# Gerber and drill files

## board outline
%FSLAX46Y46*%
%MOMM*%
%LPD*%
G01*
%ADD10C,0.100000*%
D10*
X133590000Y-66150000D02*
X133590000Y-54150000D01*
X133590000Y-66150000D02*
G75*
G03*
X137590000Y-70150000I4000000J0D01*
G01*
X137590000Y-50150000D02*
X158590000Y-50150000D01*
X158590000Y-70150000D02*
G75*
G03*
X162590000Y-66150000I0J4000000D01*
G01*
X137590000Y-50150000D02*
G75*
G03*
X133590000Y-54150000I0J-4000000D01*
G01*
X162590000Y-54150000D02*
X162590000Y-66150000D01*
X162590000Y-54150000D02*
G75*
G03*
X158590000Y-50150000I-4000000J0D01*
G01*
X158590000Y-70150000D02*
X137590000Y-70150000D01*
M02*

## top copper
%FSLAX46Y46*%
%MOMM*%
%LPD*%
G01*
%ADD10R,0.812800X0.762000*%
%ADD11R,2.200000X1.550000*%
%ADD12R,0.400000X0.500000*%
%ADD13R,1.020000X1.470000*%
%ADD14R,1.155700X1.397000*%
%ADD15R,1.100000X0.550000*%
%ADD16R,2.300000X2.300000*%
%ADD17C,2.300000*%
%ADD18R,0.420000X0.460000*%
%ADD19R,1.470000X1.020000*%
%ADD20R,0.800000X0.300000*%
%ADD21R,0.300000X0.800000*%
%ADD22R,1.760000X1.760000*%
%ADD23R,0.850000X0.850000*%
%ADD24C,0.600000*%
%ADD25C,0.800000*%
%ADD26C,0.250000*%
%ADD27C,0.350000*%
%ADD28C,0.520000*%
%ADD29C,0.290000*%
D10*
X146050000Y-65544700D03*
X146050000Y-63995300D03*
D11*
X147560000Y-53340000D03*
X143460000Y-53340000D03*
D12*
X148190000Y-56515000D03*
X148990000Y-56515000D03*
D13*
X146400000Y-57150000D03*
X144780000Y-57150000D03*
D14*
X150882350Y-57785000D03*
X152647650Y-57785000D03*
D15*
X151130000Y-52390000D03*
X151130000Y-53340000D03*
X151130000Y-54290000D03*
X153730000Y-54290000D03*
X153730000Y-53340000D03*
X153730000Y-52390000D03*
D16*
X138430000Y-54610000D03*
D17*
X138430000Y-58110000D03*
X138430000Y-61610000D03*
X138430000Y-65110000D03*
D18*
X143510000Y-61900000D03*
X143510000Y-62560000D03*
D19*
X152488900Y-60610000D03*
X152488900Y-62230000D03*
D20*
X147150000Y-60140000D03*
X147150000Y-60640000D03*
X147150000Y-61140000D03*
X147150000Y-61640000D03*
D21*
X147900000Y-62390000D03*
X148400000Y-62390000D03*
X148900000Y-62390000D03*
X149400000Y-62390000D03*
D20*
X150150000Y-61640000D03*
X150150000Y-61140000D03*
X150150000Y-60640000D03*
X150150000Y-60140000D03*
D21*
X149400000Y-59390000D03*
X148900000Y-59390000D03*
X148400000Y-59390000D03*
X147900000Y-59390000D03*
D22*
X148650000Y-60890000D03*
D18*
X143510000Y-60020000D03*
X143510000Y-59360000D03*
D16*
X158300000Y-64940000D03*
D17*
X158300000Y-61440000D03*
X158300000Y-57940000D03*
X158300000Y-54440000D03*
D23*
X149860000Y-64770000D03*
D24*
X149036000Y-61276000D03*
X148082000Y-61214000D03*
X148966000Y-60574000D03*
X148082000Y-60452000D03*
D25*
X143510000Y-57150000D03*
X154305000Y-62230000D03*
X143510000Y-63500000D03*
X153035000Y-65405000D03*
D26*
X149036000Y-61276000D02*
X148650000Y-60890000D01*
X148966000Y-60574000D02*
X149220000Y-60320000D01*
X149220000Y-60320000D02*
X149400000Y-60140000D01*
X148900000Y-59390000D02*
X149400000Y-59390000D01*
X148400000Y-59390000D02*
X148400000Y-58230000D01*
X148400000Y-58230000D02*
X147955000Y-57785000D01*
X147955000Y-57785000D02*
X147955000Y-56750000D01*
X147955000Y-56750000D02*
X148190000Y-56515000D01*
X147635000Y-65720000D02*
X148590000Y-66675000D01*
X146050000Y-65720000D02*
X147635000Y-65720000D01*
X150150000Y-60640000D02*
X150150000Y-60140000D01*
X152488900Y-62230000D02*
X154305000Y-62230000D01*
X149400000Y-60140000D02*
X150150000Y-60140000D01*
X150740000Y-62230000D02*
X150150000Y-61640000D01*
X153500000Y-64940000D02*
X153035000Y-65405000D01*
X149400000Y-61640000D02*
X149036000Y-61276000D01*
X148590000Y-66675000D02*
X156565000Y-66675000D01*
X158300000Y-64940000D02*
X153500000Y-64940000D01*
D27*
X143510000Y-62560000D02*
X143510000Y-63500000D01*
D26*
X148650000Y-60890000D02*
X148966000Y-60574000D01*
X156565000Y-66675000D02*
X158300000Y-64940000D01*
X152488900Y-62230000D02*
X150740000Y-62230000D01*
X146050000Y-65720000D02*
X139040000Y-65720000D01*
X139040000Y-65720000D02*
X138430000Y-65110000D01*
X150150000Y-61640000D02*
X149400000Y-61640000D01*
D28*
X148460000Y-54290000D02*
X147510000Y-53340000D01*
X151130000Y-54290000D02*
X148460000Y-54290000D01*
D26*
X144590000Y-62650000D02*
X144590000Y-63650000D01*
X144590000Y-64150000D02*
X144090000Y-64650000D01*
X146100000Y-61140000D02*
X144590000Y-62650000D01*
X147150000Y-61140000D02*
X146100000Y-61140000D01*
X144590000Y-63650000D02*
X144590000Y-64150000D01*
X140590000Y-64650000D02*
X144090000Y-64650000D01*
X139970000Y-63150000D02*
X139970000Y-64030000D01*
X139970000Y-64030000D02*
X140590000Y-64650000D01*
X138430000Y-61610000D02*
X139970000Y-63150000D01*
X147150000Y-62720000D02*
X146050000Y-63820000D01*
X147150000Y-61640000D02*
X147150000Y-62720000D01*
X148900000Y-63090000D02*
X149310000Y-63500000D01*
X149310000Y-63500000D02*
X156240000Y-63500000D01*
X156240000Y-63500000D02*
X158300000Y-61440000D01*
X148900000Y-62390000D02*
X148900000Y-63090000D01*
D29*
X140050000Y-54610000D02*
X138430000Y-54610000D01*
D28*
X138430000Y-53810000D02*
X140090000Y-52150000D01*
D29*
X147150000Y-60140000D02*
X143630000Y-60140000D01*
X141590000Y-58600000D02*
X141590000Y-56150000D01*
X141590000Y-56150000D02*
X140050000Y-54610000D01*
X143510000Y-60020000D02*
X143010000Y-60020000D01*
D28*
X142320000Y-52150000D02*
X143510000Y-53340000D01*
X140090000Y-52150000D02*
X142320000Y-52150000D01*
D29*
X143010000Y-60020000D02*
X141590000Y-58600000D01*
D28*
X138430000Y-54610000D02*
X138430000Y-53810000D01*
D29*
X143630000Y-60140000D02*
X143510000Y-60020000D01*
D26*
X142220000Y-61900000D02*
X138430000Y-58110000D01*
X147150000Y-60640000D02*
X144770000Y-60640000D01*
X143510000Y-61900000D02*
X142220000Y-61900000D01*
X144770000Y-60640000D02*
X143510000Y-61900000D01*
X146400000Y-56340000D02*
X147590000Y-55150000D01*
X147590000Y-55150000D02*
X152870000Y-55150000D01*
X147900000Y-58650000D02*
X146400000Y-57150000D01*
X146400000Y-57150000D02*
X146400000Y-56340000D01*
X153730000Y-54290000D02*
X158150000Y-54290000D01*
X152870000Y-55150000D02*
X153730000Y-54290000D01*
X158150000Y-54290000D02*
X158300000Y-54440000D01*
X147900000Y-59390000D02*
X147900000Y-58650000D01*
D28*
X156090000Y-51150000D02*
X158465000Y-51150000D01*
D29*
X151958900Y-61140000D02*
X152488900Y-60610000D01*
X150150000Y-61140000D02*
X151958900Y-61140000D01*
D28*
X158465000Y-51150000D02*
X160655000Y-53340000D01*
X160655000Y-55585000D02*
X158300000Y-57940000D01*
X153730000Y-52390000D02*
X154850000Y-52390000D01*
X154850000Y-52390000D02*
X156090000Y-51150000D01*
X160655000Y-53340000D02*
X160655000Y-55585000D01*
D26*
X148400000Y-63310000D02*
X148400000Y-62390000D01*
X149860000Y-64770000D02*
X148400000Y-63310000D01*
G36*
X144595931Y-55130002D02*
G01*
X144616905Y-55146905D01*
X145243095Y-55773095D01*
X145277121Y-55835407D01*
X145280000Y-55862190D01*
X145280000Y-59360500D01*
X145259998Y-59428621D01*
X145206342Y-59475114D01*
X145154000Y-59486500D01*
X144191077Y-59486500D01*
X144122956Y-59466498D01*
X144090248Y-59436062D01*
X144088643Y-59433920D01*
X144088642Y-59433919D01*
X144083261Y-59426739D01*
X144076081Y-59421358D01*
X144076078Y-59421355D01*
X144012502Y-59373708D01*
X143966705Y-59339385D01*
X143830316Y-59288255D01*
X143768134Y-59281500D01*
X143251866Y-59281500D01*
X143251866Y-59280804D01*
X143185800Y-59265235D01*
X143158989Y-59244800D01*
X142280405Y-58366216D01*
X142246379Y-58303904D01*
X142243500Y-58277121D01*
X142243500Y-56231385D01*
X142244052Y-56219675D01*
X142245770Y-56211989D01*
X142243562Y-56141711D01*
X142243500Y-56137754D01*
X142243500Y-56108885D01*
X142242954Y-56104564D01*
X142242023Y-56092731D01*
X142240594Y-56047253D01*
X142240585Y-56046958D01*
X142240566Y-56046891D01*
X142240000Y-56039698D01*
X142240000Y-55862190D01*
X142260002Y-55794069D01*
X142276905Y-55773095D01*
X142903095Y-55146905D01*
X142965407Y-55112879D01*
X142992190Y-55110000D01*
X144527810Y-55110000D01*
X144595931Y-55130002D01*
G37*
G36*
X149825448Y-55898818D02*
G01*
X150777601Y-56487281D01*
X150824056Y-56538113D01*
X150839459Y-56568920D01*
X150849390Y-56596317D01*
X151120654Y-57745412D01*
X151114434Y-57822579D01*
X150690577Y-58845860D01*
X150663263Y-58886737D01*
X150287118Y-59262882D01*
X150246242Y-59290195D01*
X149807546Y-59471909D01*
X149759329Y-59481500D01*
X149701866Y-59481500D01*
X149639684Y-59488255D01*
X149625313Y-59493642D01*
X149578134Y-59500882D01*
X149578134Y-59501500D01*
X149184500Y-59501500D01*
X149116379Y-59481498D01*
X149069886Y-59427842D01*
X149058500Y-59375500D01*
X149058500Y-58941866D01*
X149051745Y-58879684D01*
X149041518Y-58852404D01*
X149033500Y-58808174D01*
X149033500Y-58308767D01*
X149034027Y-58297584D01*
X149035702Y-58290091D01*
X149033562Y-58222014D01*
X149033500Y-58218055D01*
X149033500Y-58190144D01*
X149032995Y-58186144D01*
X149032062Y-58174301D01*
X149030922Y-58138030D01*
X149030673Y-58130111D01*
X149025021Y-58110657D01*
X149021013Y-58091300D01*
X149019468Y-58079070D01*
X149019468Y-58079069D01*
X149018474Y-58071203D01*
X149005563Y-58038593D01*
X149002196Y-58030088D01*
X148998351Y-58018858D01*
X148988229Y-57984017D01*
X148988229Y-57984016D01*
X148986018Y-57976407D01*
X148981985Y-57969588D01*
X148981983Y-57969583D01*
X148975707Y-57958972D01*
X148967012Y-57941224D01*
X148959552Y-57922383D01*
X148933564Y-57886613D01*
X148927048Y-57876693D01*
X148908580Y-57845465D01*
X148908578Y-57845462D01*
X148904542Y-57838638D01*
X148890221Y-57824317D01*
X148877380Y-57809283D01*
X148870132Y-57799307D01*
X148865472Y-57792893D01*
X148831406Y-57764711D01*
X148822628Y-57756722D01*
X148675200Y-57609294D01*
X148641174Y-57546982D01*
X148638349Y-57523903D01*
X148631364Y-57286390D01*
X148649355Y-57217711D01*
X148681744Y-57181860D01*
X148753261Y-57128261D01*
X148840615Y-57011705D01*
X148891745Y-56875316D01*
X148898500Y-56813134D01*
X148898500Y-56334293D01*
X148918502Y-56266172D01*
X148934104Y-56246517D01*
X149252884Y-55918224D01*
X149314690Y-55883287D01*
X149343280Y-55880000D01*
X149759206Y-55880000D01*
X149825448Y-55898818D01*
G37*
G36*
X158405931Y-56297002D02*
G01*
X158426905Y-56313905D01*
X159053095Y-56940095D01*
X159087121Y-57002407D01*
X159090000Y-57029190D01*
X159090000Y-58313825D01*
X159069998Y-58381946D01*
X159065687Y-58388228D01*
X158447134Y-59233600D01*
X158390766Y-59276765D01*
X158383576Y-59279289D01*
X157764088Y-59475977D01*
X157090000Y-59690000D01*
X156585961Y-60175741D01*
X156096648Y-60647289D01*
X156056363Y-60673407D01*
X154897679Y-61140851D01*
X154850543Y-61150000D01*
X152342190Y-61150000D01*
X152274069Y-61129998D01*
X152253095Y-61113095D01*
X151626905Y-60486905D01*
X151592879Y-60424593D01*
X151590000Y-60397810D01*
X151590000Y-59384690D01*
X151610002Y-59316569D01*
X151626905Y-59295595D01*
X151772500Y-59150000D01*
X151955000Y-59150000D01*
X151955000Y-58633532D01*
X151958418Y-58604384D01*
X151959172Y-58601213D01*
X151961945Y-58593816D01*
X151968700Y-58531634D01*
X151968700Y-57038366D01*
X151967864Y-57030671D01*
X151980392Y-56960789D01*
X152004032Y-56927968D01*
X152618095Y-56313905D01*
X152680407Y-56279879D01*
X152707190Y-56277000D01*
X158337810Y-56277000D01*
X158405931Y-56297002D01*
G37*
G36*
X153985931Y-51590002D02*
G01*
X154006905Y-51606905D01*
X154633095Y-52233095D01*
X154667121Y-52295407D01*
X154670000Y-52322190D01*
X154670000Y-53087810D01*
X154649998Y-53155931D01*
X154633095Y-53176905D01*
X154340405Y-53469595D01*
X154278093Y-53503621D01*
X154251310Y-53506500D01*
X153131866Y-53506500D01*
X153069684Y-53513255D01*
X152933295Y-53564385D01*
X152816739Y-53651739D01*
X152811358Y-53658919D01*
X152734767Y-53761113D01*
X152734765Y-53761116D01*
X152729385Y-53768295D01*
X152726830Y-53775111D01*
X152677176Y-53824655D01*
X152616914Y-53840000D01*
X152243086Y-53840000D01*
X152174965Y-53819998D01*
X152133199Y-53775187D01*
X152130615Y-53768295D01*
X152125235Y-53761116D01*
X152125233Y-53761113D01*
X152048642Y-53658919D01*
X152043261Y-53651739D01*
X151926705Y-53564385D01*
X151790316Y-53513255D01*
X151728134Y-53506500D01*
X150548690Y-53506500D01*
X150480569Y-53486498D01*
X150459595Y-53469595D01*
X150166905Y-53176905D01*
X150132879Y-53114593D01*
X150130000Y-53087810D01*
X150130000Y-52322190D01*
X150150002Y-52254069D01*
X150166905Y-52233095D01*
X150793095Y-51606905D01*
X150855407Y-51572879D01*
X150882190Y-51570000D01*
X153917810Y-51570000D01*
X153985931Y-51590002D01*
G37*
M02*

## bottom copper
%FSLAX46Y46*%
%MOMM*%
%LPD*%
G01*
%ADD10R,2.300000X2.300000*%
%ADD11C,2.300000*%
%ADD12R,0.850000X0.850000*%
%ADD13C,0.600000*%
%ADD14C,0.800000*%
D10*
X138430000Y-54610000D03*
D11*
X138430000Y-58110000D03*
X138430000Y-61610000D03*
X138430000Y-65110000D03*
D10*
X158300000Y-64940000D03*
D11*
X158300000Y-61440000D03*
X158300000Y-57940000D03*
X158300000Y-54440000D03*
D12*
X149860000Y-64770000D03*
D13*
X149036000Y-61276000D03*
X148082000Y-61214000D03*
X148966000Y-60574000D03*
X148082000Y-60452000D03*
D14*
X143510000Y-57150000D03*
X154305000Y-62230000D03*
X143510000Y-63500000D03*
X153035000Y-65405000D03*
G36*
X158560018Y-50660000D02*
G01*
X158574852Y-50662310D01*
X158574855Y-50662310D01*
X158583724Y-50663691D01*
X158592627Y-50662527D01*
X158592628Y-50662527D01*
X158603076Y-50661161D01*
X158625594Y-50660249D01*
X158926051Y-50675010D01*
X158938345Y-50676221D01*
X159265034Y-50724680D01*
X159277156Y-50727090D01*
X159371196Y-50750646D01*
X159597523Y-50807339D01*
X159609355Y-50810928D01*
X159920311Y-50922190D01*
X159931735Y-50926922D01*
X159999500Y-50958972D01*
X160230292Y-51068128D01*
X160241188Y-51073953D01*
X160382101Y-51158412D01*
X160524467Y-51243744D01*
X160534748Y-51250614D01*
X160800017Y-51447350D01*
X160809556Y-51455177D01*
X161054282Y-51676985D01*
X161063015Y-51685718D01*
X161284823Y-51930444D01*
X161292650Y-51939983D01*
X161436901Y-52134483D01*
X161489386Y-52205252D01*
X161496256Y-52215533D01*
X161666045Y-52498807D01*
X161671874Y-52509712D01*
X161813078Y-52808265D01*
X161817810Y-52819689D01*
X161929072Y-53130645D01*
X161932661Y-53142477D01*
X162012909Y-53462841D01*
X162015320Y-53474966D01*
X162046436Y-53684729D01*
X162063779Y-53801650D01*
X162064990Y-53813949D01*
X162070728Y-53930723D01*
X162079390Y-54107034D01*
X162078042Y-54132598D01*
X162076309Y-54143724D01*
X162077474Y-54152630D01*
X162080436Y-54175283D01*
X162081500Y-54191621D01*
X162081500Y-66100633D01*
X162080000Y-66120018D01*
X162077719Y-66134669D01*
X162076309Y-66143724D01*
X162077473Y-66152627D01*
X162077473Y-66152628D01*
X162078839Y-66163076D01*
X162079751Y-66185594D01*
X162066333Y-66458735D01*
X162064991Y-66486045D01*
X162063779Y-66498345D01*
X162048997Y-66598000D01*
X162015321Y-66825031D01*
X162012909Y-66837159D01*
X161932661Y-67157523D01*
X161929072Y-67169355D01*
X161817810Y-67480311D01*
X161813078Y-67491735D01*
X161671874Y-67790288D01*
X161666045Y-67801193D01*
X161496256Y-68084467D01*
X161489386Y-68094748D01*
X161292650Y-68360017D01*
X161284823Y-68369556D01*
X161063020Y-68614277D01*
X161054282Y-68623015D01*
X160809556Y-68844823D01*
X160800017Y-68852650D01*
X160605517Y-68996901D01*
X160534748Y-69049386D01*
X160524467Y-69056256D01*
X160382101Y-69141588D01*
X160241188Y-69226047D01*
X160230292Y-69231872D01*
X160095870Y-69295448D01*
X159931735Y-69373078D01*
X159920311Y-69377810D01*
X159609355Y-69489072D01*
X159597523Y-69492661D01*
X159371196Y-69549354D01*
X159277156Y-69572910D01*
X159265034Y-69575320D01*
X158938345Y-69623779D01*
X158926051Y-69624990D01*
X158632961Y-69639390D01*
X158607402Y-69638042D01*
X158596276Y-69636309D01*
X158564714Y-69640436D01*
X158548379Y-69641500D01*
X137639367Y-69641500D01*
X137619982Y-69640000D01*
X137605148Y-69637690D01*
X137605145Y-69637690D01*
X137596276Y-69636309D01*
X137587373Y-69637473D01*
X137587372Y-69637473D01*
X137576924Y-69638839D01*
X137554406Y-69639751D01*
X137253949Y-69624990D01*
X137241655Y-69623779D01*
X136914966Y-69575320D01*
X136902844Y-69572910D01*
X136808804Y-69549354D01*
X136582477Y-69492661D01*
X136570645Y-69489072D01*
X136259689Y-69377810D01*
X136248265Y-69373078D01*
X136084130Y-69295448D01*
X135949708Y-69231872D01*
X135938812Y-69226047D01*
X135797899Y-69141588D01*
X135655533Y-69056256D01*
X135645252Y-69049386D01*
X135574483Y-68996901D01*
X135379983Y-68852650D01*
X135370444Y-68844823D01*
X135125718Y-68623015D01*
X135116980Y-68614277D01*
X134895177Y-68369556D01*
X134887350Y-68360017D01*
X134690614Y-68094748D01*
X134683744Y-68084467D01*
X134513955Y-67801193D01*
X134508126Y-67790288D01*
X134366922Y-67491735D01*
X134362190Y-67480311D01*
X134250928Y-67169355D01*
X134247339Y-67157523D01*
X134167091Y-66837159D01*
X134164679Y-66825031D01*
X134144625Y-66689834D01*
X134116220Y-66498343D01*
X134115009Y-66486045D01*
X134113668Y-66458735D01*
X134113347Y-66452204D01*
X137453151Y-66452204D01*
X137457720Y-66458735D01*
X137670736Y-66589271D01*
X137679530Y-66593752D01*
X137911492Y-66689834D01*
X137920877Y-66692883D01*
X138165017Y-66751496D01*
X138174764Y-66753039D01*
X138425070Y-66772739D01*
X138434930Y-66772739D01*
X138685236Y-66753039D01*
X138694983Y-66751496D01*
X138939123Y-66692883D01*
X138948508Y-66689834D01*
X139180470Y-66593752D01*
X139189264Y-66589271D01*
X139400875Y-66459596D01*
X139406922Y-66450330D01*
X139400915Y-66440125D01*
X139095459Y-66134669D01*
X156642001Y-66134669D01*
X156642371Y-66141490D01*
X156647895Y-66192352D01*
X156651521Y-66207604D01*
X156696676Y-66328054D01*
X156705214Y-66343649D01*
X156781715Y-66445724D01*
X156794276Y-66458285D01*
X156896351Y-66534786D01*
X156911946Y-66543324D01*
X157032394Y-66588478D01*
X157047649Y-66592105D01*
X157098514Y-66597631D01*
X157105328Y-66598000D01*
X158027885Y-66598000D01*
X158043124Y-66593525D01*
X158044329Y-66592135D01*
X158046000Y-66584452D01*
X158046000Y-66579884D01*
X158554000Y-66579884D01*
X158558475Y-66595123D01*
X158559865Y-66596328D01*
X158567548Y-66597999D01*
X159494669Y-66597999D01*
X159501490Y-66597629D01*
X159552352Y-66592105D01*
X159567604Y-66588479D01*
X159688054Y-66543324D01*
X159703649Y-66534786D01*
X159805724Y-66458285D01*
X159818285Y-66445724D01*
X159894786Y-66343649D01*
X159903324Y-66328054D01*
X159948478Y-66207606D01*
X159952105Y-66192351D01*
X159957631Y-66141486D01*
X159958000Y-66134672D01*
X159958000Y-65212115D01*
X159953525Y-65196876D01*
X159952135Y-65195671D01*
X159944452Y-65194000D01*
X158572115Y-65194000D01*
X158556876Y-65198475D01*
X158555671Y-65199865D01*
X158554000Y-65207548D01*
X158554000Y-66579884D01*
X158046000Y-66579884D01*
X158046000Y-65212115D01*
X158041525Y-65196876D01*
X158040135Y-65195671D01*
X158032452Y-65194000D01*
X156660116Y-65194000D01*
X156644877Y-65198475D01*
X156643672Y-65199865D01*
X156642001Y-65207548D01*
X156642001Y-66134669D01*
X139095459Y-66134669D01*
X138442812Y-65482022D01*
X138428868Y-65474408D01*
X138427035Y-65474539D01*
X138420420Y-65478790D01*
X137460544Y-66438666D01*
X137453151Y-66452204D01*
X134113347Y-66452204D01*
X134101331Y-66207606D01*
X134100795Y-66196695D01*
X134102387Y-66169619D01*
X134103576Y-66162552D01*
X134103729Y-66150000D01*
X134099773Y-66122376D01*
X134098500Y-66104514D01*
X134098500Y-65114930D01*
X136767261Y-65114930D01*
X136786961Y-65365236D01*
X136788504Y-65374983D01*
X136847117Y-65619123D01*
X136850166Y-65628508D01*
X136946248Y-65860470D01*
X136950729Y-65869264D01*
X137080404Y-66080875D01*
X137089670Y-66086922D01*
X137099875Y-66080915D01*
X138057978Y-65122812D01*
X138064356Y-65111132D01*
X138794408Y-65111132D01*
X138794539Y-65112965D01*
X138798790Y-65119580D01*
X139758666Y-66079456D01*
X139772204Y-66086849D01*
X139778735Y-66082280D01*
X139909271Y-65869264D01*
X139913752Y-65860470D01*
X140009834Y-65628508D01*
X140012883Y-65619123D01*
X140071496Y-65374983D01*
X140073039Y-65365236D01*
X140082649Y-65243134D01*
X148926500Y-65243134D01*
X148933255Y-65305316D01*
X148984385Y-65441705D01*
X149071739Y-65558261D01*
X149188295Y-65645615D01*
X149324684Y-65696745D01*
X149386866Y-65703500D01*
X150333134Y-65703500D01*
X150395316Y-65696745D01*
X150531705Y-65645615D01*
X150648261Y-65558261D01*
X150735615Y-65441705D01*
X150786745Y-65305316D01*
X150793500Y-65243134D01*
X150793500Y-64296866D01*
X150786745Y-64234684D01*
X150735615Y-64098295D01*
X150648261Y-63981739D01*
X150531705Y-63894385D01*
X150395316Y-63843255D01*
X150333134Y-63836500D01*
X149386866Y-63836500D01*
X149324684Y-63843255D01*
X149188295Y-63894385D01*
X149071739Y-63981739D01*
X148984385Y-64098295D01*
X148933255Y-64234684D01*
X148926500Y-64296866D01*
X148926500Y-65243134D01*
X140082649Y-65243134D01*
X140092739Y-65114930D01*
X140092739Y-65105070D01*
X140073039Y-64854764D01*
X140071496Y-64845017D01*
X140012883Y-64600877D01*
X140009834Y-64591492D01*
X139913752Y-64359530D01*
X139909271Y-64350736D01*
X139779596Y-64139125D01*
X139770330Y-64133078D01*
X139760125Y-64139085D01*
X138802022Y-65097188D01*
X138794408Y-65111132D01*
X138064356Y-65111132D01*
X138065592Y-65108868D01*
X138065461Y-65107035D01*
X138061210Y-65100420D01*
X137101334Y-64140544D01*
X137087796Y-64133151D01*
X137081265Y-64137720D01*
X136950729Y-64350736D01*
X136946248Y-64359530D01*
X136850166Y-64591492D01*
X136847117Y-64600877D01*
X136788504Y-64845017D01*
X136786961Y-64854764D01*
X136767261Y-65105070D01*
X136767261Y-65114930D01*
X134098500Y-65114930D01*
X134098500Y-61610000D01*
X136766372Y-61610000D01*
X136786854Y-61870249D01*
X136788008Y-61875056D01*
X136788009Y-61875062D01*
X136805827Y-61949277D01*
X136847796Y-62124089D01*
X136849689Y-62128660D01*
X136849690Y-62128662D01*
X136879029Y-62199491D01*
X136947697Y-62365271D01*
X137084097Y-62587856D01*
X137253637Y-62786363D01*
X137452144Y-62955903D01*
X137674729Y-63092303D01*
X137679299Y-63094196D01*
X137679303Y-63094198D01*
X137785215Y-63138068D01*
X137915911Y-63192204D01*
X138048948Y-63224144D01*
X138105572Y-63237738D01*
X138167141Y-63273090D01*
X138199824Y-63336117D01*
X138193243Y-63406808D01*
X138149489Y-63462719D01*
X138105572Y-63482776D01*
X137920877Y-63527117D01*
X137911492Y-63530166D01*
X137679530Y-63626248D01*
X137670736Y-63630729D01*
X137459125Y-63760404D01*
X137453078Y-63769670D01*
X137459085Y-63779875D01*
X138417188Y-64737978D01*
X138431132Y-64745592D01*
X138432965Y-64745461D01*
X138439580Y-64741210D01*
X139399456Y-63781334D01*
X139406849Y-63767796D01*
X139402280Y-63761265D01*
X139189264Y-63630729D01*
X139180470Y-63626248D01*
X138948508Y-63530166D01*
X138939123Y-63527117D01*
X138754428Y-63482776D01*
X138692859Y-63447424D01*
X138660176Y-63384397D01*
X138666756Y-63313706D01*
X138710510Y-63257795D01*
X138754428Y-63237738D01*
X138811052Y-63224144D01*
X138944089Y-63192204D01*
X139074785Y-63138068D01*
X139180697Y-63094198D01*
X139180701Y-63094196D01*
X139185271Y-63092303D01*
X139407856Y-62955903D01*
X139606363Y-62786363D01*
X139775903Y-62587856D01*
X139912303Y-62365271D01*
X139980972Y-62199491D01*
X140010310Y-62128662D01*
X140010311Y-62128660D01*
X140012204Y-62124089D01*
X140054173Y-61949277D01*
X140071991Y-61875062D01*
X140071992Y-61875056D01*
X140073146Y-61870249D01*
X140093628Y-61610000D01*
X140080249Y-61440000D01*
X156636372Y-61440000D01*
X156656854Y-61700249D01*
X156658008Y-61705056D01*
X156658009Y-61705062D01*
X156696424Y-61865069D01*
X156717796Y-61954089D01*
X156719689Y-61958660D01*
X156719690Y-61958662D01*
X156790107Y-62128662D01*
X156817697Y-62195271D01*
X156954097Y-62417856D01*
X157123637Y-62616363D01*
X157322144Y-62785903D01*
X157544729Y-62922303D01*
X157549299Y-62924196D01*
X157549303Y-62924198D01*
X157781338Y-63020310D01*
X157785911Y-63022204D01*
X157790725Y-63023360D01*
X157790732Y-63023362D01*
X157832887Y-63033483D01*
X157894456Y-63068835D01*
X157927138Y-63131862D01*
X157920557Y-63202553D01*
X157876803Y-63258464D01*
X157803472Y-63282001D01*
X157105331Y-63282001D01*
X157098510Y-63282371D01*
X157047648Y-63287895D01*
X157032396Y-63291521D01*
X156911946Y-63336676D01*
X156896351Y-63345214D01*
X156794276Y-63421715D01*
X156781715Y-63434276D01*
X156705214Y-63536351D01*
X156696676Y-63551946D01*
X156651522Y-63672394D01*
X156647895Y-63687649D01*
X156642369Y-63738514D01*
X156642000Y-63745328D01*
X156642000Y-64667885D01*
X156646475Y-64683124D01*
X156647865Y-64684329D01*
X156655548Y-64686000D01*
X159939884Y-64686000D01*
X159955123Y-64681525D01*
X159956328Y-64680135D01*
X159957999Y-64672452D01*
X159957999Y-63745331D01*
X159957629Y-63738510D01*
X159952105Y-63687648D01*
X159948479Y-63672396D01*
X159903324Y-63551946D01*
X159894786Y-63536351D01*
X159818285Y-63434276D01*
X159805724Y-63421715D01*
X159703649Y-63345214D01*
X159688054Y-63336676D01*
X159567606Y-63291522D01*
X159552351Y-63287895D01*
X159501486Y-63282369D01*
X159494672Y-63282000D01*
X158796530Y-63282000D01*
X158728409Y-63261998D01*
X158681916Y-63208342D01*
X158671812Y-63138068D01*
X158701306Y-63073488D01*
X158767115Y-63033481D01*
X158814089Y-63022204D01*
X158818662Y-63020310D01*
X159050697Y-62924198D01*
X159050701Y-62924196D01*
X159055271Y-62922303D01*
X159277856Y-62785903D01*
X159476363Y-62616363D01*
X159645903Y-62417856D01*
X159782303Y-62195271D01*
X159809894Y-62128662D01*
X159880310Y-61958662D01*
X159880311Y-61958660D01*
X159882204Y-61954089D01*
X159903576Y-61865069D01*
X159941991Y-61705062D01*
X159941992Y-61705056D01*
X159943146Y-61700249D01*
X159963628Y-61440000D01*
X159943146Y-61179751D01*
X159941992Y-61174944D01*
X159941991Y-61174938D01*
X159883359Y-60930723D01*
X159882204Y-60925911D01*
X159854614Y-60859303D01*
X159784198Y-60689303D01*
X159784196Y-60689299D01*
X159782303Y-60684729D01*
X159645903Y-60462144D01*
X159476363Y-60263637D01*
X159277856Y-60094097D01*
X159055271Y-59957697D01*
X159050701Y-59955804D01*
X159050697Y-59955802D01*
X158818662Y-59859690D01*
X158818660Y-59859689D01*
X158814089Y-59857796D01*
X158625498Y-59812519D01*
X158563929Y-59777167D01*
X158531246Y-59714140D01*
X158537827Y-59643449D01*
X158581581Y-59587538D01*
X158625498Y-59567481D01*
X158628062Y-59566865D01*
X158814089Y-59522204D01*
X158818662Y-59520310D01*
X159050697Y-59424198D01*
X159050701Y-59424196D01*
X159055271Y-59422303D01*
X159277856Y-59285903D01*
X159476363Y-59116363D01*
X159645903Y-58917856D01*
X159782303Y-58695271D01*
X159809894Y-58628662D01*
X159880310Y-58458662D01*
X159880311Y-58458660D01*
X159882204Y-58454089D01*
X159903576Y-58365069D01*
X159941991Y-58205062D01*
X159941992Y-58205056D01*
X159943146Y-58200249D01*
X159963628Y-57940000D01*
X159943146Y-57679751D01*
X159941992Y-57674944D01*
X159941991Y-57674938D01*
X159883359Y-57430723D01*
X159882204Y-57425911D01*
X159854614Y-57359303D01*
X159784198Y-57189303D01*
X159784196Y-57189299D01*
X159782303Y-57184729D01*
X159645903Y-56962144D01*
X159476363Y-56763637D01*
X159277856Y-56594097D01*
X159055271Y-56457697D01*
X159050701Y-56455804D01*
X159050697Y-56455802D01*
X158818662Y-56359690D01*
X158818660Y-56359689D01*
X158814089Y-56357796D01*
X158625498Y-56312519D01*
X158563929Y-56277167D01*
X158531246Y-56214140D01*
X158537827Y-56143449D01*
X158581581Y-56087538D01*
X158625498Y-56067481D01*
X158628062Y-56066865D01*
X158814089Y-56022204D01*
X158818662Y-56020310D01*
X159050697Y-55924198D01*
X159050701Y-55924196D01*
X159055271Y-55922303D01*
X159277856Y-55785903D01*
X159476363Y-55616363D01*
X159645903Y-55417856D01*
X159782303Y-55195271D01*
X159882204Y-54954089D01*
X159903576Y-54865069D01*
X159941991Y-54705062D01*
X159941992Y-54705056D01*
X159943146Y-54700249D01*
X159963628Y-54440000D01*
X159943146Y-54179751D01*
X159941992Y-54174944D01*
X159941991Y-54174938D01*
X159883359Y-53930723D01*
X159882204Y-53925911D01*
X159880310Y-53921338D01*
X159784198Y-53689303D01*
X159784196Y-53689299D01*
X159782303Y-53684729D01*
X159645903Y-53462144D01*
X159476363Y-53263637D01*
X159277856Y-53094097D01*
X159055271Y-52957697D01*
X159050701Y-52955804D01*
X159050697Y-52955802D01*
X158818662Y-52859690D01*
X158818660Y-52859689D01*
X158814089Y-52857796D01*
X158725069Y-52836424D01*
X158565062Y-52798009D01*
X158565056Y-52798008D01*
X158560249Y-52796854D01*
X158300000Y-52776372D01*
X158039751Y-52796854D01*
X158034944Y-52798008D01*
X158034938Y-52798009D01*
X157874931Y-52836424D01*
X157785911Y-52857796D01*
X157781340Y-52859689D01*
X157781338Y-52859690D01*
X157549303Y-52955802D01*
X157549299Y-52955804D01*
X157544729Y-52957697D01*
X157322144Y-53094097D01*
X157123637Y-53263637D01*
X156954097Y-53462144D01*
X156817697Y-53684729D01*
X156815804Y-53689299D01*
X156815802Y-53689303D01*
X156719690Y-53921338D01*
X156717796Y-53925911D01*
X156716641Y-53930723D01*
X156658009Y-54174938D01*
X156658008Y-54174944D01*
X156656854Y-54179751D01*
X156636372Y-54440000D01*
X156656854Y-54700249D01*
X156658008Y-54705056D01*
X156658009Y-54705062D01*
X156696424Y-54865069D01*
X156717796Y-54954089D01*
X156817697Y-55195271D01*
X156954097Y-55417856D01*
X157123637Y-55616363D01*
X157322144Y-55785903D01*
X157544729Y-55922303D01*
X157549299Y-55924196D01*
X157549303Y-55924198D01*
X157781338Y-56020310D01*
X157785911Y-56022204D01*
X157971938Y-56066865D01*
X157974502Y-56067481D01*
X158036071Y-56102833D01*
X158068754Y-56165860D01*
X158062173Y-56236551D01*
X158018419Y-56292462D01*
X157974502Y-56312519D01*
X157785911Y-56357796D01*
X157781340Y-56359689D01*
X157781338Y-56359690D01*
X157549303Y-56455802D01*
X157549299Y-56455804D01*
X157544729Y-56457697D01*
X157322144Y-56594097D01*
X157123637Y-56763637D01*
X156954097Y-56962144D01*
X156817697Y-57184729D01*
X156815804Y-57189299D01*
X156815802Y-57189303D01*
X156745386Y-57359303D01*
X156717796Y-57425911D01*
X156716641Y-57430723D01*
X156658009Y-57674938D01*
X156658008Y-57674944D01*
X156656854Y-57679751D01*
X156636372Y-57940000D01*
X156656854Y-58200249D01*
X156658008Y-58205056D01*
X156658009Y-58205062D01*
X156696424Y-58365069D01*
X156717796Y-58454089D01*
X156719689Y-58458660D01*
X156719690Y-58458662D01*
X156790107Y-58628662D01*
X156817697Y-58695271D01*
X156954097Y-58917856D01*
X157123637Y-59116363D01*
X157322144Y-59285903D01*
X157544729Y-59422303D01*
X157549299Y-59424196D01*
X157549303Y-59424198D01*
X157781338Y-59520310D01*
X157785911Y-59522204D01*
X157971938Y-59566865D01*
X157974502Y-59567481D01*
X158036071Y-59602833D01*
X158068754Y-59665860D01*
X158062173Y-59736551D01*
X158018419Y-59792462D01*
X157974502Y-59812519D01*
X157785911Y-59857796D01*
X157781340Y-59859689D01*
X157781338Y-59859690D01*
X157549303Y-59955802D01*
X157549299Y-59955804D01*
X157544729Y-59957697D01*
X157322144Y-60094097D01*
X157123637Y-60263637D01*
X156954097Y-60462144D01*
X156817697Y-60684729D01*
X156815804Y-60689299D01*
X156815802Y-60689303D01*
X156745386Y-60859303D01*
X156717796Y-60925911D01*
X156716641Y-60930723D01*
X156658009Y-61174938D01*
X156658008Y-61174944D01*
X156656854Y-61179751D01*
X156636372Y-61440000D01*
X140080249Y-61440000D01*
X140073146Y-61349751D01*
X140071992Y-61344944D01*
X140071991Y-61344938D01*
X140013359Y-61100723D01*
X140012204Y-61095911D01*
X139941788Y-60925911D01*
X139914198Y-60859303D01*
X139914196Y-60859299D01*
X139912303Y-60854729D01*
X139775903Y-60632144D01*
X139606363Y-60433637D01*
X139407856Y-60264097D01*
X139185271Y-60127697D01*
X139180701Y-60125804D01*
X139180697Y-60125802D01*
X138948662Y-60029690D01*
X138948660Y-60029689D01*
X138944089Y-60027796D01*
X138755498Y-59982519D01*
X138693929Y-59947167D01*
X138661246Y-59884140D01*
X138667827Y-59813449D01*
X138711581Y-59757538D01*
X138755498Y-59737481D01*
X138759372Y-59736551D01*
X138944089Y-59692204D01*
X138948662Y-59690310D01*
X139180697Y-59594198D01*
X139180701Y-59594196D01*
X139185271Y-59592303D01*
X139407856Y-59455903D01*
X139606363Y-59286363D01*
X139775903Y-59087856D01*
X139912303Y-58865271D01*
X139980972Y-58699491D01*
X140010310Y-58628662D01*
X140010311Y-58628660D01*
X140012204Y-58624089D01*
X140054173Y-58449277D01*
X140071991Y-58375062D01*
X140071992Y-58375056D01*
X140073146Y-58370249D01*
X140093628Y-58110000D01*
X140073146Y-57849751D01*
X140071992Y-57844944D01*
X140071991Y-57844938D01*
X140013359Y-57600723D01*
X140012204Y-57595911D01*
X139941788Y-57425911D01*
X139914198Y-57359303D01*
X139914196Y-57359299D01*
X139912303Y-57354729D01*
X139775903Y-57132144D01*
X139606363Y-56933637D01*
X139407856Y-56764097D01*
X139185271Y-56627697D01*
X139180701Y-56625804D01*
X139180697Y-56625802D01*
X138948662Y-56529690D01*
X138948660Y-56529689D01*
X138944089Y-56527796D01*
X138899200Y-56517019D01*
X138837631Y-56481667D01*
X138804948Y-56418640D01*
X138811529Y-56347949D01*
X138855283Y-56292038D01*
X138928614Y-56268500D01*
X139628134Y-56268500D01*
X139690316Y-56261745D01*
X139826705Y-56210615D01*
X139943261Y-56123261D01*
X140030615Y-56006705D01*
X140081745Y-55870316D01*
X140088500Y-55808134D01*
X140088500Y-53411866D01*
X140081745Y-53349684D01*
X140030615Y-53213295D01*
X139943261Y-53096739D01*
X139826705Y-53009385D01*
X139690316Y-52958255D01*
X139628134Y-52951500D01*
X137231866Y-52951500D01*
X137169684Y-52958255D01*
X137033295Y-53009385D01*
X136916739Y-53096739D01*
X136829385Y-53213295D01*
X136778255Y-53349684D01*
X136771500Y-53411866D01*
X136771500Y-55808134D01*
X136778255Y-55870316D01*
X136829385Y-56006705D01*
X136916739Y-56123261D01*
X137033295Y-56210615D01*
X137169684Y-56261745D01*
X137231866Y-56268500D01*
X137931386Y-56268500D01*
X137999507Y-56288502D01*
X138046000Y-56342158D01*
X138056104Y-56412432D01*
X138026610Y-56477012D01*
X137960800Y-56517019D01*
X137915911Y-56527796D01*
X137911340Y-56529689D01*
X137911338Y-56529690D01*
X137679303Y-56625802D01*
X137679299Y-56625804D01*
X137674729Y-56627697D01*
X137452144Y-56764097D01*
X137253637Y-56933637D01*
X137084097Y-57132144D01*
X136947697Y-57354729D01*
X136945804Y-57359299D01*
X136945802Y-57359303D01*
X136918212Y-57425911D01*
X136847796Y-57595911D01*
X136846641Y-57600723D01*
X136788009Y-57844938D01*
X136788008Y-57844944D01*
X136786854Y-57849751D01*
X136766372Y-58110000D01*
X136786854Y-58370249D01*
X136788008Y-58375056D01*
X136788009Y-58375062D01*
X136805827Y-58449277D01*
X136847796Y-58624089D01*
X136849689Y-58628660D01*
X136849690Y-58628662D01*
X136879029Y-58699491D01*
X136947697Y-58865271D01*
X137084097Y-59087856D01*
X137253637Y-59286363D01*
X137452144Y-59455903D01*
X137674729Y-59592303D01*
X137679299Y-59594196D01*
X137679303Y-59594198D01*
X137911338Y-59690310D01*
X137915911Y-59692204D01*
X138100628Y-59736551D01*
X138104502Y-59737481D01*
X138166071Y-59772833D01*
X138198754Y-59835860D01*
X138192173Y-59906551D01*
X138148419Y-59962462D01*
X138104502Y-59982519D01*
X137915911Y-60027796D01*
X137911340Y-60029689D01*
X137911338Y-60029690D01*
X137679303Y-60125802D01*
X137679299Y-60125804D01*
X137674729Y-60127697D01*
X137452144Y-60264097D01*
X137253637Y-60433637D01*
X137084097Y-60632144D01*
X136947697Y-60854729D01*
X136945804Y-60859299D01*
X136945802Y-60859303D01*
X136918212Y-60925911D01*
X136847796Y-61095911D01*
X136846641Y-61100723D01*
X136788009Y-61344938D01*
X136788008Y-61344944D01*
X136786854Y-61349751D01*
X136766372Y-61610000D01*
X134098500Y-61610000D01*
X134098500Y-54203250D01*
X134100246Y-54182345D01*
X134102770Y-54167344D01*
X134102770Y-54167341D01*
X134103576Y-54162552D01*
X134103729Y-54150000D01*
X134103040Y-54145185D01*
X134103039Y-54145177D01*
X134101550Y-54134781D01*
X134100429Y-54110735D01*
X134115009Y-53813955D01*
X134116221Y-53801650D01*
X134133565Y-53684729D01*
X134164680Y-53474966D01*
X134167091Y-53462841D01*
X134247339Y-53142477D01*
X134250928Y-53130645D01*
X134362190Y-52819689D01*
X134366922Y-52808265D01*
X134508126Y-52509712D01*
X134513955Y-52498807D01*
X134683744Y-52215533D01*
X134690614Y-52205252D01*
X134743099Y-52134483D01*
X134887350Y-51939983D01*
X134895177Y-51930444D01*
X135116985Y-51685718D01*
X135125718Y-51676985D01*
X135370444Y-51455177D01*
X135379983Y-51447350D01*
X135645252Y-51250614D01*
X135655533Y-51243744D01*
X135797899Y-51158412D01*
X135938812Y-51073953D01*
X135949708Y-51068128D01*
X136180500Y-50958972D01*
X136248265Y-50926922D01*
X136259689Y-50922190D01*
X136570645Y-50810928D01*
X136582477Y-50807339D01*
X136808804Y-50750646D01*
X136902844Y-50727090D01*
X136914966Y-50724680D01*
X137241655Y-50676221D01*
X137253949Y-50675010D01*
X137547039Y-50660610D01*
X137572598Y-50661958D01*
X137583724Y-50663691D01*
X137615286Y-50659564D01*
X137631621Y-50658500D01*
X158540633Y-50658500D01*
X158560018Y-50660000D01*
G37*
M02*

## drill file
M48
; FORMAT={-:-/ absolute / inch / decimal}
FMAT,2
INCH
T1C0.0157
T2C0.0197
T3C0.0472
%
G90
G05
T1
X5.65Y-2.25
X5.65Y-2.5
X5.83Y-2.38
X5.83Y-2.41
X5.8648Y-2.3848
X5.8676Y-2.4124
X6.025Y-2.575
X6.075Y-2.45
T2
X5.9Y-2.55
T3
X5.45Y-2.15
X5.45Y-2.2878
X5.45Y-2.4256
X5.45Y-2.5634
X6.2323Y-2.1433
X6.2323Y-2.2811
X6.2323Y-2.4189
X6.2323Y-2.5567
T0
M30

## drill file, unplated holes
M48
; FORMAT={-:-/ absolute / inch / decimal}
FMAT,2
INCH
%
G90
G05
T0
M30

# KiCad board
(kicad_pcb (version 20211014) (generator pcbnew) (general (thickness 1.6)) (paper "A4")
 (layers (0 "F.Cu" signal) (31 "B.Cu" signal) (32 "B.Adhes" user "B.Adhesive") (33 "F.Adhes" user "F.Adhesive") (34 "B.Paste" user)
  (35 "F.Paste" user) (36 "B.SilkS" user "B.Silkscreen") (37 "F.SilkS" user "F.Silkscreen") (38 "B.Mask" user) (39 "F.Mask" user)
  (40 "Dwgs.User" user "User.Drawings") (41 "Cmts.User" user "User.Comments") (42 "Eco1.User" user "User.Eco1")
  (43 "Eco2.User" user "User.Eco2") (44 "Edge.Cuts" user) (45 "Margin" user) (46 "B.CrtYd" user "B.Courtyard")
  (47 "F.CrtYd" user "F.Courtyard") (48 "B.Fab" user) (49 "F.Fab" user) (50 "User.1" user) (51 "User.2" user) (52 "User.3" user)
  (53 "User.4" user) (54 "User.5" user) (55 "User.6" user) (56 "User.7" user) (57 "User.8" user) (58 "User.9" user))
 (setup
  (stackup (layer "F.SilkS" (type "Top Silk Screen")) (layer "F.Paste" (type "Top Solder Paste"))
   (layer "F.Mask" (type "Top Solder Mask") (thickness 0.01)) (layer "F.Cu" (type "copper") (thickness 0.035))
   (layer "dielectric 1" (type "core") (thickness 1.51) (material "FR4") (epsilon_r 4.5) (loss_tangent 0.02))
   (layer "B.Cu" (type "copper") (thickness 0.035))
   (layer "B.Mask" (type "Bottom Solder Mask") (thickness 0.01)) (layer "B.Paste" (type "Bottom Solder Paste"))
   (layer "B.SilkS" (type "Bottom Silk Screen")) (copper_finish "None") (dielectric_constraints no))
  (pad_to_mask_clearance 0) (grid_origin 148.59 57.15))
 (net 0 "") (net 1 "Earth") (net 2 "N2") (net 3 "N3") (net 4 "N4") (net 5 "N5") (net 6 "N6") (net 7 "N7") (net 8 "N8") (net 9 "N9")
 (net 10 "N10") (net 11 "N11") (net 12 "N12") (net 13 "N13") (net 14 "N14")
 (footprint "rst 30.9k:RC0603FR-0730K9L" (layer "F.Cu") (at 146.05 64.77 90)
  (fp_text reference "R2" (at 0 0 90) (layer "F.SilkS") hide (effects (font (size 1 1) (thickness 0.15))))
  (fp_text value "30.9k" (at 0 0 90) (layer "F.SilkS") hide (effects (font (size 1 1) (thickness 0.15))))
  (pad "1" smd rect (at -0.7747 0 90) (size 0.762 0.8128) (layers "F.Cu" "F.Paste" "F.Mask") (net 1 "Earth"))
  (pad "2" smd rect (at 0.7747 0 90) (size 0.762 0.8128) (layers "F.Cu" "F.Paste" "F.Mask") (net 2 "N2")))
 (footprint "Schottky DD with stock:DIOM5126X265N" (layer "F.Cu") (at 145.51 53.34 180)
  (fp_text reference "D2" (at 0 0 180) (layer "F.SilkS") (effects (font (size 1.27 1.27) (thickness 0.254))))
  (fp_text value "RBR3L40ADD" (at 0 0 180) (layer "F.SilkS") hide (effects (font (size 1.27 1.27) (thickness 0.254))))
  (pad "1" smd rect (at -2.05 0 270) (size 1.55 2.2) (layers "F.Cu" "F.Paste" "F.Mask") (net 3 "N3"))
  (pad "2" smd rect (at 2.05 0 270) (size 1.55 2.2) (layers "F.Cu" "F.Paste" "F.Mask") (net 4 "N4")))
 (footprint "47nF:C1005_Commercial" (layer "F.Cu") (at 148.59 56.515)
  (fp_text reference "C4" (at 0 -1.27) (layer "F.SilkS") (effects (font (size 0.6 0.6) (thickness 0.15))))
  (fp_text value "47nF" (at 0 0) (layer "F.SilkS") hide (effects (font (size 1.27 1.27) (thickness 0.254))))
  (pad "1" smd rect (at -0.4 0) (size 0.4 0.5) (layers "F.Cu" "F.Paste" "F.Mask") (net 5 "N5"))
  (pad "2" smd rect (at 0.4 0) (size 0.4 0.5) (layers "F.Cu" "F.Paste" "F.Mask") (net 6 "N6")))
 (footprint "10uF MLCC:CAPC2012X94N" (layer "F.Cu") (at 145.59 57.15 180)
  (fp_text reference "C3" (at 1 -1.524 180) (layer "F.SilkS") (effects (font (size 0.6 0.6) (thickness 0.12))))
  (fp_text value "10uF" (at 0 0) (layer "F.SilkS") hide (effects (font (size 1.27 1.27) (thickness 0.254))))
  (pad "1" smd rect (at -0.81 0 180) (size 1.02 1.47) (layers "F.Cu" "F.Paste" "F.Mask") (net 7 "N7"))
  (pad "2" smd rect (at 0.81 0 180) (size 1.02 1.47) (layers "F.Cu" "F.Paste" "F.Mask") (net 1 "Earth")))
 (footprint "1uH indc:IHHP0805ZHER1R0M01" (layer "F.Cu") (at 151.765 57.785)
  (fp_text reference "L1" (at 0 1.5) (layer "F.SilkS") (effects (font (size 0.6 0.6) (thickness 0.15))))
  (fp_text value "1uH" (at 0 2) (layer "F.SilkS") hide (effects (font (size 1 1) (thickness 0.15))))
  (pad "1" smd rect (at -0.88265 0) (size 1.1557 1.397) (layers "F.Cu" "F.Paste" "F.Mask") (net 6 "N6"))
  (pad "2" smd rect (at 0.88265 0) (size 1.1557 1.397) (layers "F.Cu" "F.Paste" "F.Mask") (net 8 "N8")))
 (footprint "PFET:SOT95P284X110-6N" (layer "F.Cu") (at 152.43 53.34)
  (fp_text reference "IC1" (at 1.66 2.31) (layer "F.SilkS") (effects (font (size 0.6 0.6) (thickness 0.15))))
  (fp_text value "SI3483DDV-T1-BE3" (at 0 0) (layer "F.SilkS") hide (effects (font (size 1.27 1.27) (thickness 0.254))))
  (pad "1" smd rect (at -1.3 -0.95 90) (size 0.55 1.1) (layers "F.Cu" "F.Paste" "F.Mask") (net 8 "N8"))
  (pad "2" smd rect (at -1.3 0 90) (size 0.55 1.1) (layers "F.Cu" "F.Paste" "F.Mask") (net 8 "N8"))
  (pad "3" smd rect (at -1.3 0.95 90) (size 0.55 1.1) (layers "F.Cu" "F.Paste" "F.Mask") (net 3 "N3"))
  (pad "4" smd rect (at 1.3 0.95 90) (size 0.55 1.1) (layers "F.Cu" "F.Paste" "F.Mask") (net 7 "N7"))
  (pad "5" smd rect (at 1.3 0 90) (size 0.55 1.1) (layers "F.Cu" "F.Paste" "F.Mask") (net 8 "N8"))
  (pad "6" smd rect (at 1.3 -0.95 90) (size 0.55 1.1) (layers "F.Cu" "F.Paste" "F.Mask") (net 8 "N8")))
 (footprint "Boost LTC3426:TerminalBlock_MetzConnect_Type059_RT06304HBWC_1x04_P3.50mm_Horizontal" (layer "F.Cu") (at 138.43 54.61 -90)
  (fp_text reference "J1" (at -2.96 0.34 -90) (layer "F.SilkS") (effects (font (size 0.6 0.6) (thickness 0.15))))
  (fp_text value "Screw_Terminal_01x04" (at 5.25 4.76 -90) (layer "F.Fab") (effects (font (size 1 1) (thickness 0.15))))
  (pad "1" thru_hole rect (at 0 0 270) (size 2.3 2.3) (drill 1.2) (layers *.Cu *.Mask) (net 4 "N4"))
  (pad "2" thru_hole circle (at 3.5 0 270) (size 2.3 2.3) (drill 1.2) (layers *.Cu *.Mask) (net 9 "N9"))
  (pad "3" thru_hole circle (at 7 0 270) (size 2.3 2.3) (drill 1.2) (layers *.Cu *.Mask) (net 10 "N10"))
  (pad "4" thru_hole circle (at 10.5 0 270) (size 2.3 2.3) (drill 1.2) (layers *.Cu *.Mask) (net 1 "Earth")))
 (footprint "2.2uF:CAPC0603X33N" (layer "F.Cu") (at 143.51 62.23 -90)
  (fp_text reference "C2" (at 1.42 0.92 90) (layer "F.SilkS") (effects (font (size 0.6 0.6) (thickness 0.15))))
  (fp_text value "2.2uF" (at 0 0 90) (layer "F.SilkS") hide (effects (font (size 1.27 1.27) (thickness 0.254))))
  (pad "1" smd rect (at -0.33 0) (size 0.42 0.46) (layers "F.Cu" "F.Paste" "F.Mask") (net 9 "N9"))
  (pad "2" smd rect (at 0.33 0) (size 0.42 0.46) (layers "F.Cu" "F.Paste" "F.Mask") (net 1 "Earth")))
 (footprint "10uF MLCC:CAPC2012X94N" (layer "F.Cu") (at 152.4889 61.42 -90)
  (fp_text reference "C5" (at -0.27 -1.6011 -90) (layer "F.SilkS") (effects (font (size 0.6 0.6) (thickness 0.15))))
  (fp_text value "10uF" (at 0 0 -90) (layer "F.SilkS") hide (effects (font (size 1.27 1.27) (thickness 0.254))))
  (pad "1" smd rect (at -0.81 0 270) (size 1.02 1.47) (layers "F.Cu" "F.Paste" "F.Mask") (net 8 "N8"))
  (pad "2" smd rect (at 0.81 0 270) (size 1.02 1.47) (layers "F.Cu" "F.Paste" "F.Mask") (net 1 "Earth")))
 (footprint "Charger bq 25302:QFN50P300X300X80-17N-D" (layer "F.Cu") (at 148.65 60.89)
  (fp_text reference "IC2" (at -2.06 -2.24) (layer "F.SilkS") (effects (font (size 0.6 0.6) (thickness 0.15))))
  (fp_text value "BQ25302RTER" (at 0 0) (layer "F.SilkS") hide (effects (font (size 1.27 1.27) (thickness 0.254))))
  (pad "1" smd rect (at -1.5 -0.75 90) (size 0.3 0.8) (layers "F.Cu" "F.Paste" "F.Mask") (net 4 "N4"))
  (pad "2" smd rect (at -1.5 -0.25 90) (size 0.3 0.8) (layers "F.Cu" "F.Paste" "F.Mask") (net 9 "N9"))
  (pad "3" smd rect (at -1.5 0.25 90) (size 0.3 0.8) (layers "F.Cu" "F.Paste" "F.Mask") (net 10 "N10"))
  (pad "4" smd rect (at -1.5 0.75 90) (size 0.3 0.8) (layers "F.Cu" "F.Paste" "F.Mask") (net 2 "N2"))
  (pad "5" smd rect (at -0.75 1.5) (size 0.3 0.8) (layers "F.Cu" "F.Paste" "F.Mask") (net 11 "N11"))
  (pad "6" smd rect (at -0.25 1.5) (size 0.3 0.8) (layers "F.Cu" "F.Paste" "F.Mask") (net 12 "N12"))
  (pad "7" smd rect (at 0.25 1.5) (size 0.3 0.8) (layers "F.Cu" "F.Paste" "F.Mask") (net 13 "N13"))
  (pad "8" smd rect (at 0.75 1.5) (size 0.3 0.8) (layers "F.Cu" "F.Paste" "F.Mask") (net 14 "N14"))
  (pad "9" smd rect (at 1.5 0.75 90) (size 0.3 0.8) (layers "F.Cu" "F.Paste" "F.Mask") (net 1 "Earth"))
  (pad "10" smd rect (at 1.5 0.25 90) (size 0.3 0.8) (layers "F.Cu" "F.Paste" "F.Mask") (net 8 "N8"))
  (pad "11" smd rect (at 1.5 -0.25 90) (size 0.3 0.8) (layers "F.Cu" "F.Paste" "F.Mask") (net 1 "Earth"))
  (pad "12" smd rect (at 1.5 -0.75 90) (size 0.3 0.8) (layers "F.Cu" "F.Paste" "F.Mask") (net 1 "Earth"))
  (pad "13" smd rect (at 0.75 -1.5) (size 0.3 0.8) (layers "F.Cu" "F.Paste" "F.Mask") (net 6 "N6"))
  (pad "14" smd rect (at 0.25 -1.5) (size 0.3 0.8) (layers "F.Cu" "F.Paste" "F.Mask") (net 6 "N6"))
  (pad "15" smd rect (at -0.25 -1.5) (size 0.3 0.8) (layers "F.Cu" "F.Paste" "F.Mask") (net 5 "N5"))
  (pad "16" smd rect (at -0.75 -1.5) (size 0.3 0.8) (layers "F.Cu" "F.Paste" "F.Mask") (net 7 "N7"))
  (pad "17" smd rect (at 0 0) (size 1.76 1.76) (layers "F.Cu" "F.Paste" "F.Mask") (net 1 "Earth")))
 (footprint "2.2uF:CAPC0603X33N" (layer "F.Cu") (at 143.51 59.69 90)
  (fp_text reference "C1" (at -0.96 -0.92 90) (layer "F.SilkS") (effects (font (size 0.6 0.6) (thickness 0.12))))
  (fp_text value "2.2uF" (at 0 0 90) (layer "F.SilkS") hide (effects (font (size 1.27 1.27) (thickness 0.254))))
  (pad "1" smd rect (at -0.33 0 180) (size 0.42 0.46) (layers "F.Cu" "F.Paste" "F.Mask") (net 4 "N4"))
  (pad "2" smd rect (at 0.33 0 180) (size 0.42 0.46) (layers "F.Cu" "F.Paste" "F.Mask") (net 1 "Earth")))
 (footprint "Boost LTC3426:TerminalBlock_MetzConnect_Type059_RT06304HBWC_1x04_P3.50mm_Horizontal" (layer "F.Cu") (at 158.3 64.94 90)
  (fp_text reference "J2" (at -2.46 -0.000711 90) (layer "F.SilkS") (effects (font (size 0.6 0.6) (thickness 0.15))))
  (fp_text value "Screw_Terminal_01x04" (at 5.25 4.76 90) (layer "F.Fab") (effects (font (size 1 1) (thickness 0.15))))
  (pad "1" thru_hole rect (at 0 0 90) (size 2.3 2.3) (drill 1.2) (layers *.Cu *.Mask) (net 1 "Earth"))
  (pad "2" thru_hole circle (at 3.5 0 90) (size 2.3 2.3) (drill 1.2) (layers *.Cu *.Mask) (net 13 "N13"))
  (pad "3" thru_hole circle (at 7 0 90) (size 2.3 2.3) (drill 1.2) (layers *.Cu *.Mask) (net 8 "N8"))
  (pad "4" thru_hole circle (at 10.5 0 90) (size 2.3 2.3) (drill 1.2) (layers *.Cu *.Mask) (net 7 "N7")))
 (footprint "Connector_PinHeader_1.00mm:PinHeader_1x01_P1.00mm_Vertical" (layer "F.Cu") (at 149.86 64.77)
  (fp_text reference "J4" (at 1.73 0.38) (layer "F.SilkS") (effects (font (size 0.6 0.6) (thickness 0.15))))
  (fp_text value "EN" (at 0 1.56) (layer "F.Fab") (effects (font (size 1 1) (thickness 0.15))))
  (pad "1" thru_hole rect (at 0 0) (size 0.85 0.85) (drill 0.5) (layers *.Cu *.Mask) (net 12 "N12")))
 (gr_line (start 133.59 66.15) (end 133.59 54.15) (layer "Edge.Cuts") (width 0.1))
 (gr_arc (start 137.59 70.15) (mid 134.761573 68.978427) (end 133.59 66.15) (layer "Edge.Cuts") (width 0.1))
 (gr_line (start 137.59 50.15) (end 158.59 50.15) (layer "Edge.Cuts") (width 0.1))
 (gr_arc (start 162.59 66.15) (mid 161.418427 68.978427) (end 158.59 70.15) (layer "Edge.Cuts") (width 0.1))
 (gr_arc (start 133.59 54.15) (mid 134.761573 51.321573) (end 137.59 50.15) (layer "Edge.Cuts") (width 0.1))
 (gr_line (start 162.59 54.15) (end 162.59 66.15) (layer "Edge.Cuts") (width 0.1))
 (gr_arc (start 158.59 50.15) (mid 161.418427 51.321573) (end 162.59 54.15) (layer "Edge.Cuts") (width 0.1))
 (gr_line (start 158.59 70.15) (end 137.59 70.15) (layer "Edge.Cuts") (width 0.1))
 (segment (start 148.966 60.574) (end 149.22 60.32) (width 0.25) (layer "F.Cu") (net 1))
 (segment (start 147.635 65.72) (end 148.59 66.675) (width 0.25) (layer "F.Cu") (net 1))
 (segment (start 146.05 65.72) (end 147.635 65.72) (width 0.25) (layer "F.Cu") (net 1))
 (segment (start 150.15 60.64) (end 150.15 60.14) (width 0.25) (layer "F.Cu") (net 1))
 (segment (start 152.4889 62.23) (end 154.305 62.23) (width 0.25) (layer "F.Cu") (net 1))
 (segment (start 149.4 60.14) (end 150.15 60.14) (width 0.25) (layer "F.Cu") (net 1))
 (segment (start 150.74 62.23) (end 150.15 61.64) (width 0.25) (layer "F.Cu") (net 1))
 (segment (start 153.5 64.94) (end 153.035 65.405) (width 0.25) (layer "F.Cu") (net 1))
 (segment (start 149.4 61.64) (end 149.036 61.276) (width 0.25) (layer "F.Cu") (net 1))
 (segment (start 148.59 66.675) (end 156.565 66.675) (width 0.25) (layer "F.Cu") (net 1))
 (segment (start 158.3 64.94) (end 153.5 64.94) (width 0.25) (layer "F.Cu") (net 1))
 (segment (start 143.51 62.56) (end 143.51 63.5) (width 0.35) (layer "F.Cu") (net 1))
 (segment (start 148.65 60.89) (end 148.966 60.574) (width 0.25) (layer "F.Cu") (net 1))
 (segment (start 149.036 61.276) (end 148.65 60.89) (width 0.25) (layer "F.Cu") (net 1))
 (segment (start 156.565 66.675) (end 158.3 64.94) (width 0.25) (layer "F.Cu") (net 1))
 (segment (start 152.4889 62.23) (end 150.74 62.23) (width 0.25) (layer "F.Cu") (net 1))
 (segment (start 146.05 65.72) (end 139.04 65.72) (width 0.25) (layer "F.Cu") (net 1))
 (segment (start 149.22 60.32) (end 149.4 60.14) (width 0.25) (layer "F.Cu") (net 1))
 (segment (start 139.04 65.72) (end 138.43 65.11) (width 0.25) (layer "F.Cu") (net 1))
 (segment (start 150.15 61.64) (end 149.4 61.64) (width 0.25) (layer "F.Cu") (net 1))
 (via (at 149.036 61.276) (size 0.6) (drill 0.4) (layers "F.Cu" "B.Cu") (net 1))
 (via (at 143.51 57.15) (size 0.8) (drill 0.4) (layers "F.Cu" "B.Cu") (free) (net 1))
 (via (at 148.082 61.214) (size 0.6) (drill 0.4) (layers "F.Cu" "B.Cu") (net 1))
 (via (at 154.305 62.23) (size 0.8) (drill 0.4) (layers "F.Cu" "B.Cu") (free) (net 1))
 (via (at 143.51 63.5) (size 0.8) (drill 0.4) (layers "F.Cu" "B.Cu") (free) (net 1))
 (via (at 153.035 65.405) (size 0.8) (drill 0.4) (layers "F.Cu" "B.Cu") (free) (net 1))
 (via (at 148.082 60.452) (size 0.6) (drill 0.4) (layers "F.Cu" "B.Cu") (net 1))
 (via (at 148.966 60.574) (size 0.6) (drill 0.4) (layers "F.Cu" "B.Cu") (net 1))
 (segment (start 148.46 54.29) (end 147.51 53.34) (width 0.52) (layer "F.Cu") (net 3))
 (segment (start 151.13 54.29) (end 148.46 54.29) (width 0.52) (layer "F.Cu") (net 3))
 (segment (start 144.59 62.65) (end 144.59 63.65) (width 0.25) (layer "F.Cu") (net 10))
 (segment (start 144.59 64.15) (end 144.09 64.65) (width 0.25) (layer "F.Cu") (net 10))
 (segment (start 146.1 61.14) (end 144.59 62.65) (width 0.25) (layer "F.Cu") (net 10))
 (segment (start 147.15 61.14) (end 146.1 61.14) (width 0.25) (layer "F.Cu") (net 10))
 (segment (start 144.59 63.65) (end 144.59 64.15) (width 0.25) (layer "F.Cu") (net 10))
 (segment (start 140.59 64.65) (end 144.09 64.65) (width 0.25) (layer "F.Cu") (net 10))
 (segment (start 139.97 63.15) (end 139.97 64.03) (width 0.25) (layer "F.Cu") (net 10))
 (segment (start 139.97 64.03) (end 140.59 64.65) (width 0.25) (layer "F.Cu") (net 10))
 (segment (start 138.43 61.61) (end 139.97 63.15) (width 0.25) (layer "F.Cu") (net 10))
 (segment (start 147.15 62.72) (end 146.05 63.82) (width 0.25) (layer "F.Cu") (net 2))
 (segment (start 147.15 61.64) (end 147.15 62.72) (width 0.25) (layer "F.Cu") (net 2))
 (segment (start 148.9 63.09) (end 149.31 63.5) (width 0.25) (layer "F.Cu") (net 13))
 (segment (start 149.31 63.5) (end 156.24 63.5) (width 0.25) (layer "F.Cu") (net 13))
 (segment (start 156.24 63.5) (end 158.3 61.44) (width 0.25) (layer "F.Cu") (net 13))
 (segment (start 148.9 62.39) (end 148.9 63.09) (width 0.25) (layer "F.Cu") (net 13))
 (segment (start 140.05 54.61) (end 138.43 54.61) (width 0.29) (layer "F.Cu") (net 4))
 (segment (start 138.43 53.81) (end 140.09 52.15) (width 0.52) (layer "F.Cu") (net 4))
 (segment (start 147.15 60.14) (end 143.63 60.14) (width 0.29) (layer "F.Cu") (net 4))
 (segment (start 141.59 58.6) (end 141.59 56.15) (width 0.29) (layer "F.Cu") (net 4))
 (segment (start 141.59 56.15) (end 140.05 54.61) (width 0.29) (layer "F.Cu") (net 4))
 (segment (start 143.51 60.02) (end 143.01 60.02) (width 0.29) (layer "F.Cu") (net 4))
 (segment (start 142.32 52.15) (end 143.51 53.34) (width 0.52) (layer "F.Cu") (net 4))
 (segment (start 140.09 52.15) (end 142.32 52.15) (width 0.52) (layer "F.Cu") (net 4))
 (segment (start 143.01 60.02) (end 141.59 58.6) (width 0.29) (layer "F.Cu") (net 4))
 (segment (start 138.43 54.61) (end 138.43 53.81) (width 0.52) (layer "F.Cu") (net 4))
 (segment (start 143.63 60.14) (end 143.51 60.02) (width 0.29) (layer "F.Cu") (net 4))
 (segment (start 142.22 61.9) (end 138.43 58.11) (width 0.25) (layer "F.Cu") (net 9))
 (segment (start 147.15 60.64) (end 144.77 60.64) (width 0.25) (layer "F.Cu") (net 9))
 (segment (start 143.51 61.9) (end 142.22 61.9) (width 0.25) (layer "F.Cu") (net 9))
 (segment (start 144.77 60.64) (end 143.51 61.9) (width 0.25) (layer "F.Cu") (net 9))
 (segment (start 146.4 56.34) (end 147.59 55.15) (width 0.25) (layer "F.Cu") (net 7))
 (segment (start 147.59 55.15) (end 152.87 55.15) (width 0.25) (layer "F.Cu") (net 7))
 (segment (start 147.9 58.65) (end 146.4 57.15) (width 0.25) (layer "F.Cu") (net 7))
 (segment (start 146.4 57.15) (end 146.4 56.34) (width 0.25) (layer "F.Cu") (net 7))
 (segment (start 153.73 54.29) (end 158.15 54.29) (width 0.25) (layer "F.Cu") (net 7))
 (segment (start 152.87 55.15) (end 153.73 54.29) (width 0.25) (layer "F.Cu") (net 7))
 (segment (start 158.15 54.29) (end 158.3 54.44) (width 0.25) (layer "F.Cu") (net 7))
 (segment (start 147.9 59.39) (end 147.9 58.65) (width 0.25) (layer "F.Cu") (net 7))
 (segment (start 147.955 57.785) (end 147.955 56.75) (width 0.25) (layer "F.Cu") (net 5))
 (segment (start 148.4 58.23) (end 147.955 57.785) (width 0.25) (layer "F.Cu") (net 5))
 (segment (start 147.955 56.75) (end 148.19 56.515) (width 0.25) (layer "F.Cu") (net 5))
 (segment (start 148.4 59.39) (end 148.4 58.23) (width 0.25) (layer "F.Cu") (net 5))
 (segment (start 148.9 59.39) (end 149.4 59.39) (width 0.25) (layer "F.Cu") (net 6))
 (segment (start 156.09 51.15) (end 158.465 51.15) (width 0.52) (layer "F.Cu") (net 8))
 (segment (start 151.9589 61.14) (end 152.4889 60.61) (width 0.29) (layer "F.Cu") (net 8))
 (segment (start 150.15 61.14) (end 151.9589 61.14) (width 0.29) (layer "F.Cu") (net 8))
 (segment (start 158.465 51.15) (end 160.655 53.34) (width 0.52) (layer "F.Cu") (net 8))
 (segment (start 160.655 55.585) (end 158.3 57.94) (width 0.52) (layer "F.Cu") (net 8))
 (segment (start 153.73 52.39) (end 154.85 52.39) (width 0.52) (layer "F.Cu") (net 8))
 (segment (start 154.85 52.39) (end 156.09 51.15) (width 0.52) (layer "F.Cu") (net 8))
 (segment (start 160.655 53.34) (end 160.655 55.585) (width 0.52) (layer "F.Cu") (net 8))
 (segment (start 148.4 63.31) (end 148.4 62.39) (width 0.25) (layer "F.Cu") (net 12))
 (segment (start 149.86 64.77) (end 148.4 63.31) (width 0.25) (layer "F.Cu") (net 12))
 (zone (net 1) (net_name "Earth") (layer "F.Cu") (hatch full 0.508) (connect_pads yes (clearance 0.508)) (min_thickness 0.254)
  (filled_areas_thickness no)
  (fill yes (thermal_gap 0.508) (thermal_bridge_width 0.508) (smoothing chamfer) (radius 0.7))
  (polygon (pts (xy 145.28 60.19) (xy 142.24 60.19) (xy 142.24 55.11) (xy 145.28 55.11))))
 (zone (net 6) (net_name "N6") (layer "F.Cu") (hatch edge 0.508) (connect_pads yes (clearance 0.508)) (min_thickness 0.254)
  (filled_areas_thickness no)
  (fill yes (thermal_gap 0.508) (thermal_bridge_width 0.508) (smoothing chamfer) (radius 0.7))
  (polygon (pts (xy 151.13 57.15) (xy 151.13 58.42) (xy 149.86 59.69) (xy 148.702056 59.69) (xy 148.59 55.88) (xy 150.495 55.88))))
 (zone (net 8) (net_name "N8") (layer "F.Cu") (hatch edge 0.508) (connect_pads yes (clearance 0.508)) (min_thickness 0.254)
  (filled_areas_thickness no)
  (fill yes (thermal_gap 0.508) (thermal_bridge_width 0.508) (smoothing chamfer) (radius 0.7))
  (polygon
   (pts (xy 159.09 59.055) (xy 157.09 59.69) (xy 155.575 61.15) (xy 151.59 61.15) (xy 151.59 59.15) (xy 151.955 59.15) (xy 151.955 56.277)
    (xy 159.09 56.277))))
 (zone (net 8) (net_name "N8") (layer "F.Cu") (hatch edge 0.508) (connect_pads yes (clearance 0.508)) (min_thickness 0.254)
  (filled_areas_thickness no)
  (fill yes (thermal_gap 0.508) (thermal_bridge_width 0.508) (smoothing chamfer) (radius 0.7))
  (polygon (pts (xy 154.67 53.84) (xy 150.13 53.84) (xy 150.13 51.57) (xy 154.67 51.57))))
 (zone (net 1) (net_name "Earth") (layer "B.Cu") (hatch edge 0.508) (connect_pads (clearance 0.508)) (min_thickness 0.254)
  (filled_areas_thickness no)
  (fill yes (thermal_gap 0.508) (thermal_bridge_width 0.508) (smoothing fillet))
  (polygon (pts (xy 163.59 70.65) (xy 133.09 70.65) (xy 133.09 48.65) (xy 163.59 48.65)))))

